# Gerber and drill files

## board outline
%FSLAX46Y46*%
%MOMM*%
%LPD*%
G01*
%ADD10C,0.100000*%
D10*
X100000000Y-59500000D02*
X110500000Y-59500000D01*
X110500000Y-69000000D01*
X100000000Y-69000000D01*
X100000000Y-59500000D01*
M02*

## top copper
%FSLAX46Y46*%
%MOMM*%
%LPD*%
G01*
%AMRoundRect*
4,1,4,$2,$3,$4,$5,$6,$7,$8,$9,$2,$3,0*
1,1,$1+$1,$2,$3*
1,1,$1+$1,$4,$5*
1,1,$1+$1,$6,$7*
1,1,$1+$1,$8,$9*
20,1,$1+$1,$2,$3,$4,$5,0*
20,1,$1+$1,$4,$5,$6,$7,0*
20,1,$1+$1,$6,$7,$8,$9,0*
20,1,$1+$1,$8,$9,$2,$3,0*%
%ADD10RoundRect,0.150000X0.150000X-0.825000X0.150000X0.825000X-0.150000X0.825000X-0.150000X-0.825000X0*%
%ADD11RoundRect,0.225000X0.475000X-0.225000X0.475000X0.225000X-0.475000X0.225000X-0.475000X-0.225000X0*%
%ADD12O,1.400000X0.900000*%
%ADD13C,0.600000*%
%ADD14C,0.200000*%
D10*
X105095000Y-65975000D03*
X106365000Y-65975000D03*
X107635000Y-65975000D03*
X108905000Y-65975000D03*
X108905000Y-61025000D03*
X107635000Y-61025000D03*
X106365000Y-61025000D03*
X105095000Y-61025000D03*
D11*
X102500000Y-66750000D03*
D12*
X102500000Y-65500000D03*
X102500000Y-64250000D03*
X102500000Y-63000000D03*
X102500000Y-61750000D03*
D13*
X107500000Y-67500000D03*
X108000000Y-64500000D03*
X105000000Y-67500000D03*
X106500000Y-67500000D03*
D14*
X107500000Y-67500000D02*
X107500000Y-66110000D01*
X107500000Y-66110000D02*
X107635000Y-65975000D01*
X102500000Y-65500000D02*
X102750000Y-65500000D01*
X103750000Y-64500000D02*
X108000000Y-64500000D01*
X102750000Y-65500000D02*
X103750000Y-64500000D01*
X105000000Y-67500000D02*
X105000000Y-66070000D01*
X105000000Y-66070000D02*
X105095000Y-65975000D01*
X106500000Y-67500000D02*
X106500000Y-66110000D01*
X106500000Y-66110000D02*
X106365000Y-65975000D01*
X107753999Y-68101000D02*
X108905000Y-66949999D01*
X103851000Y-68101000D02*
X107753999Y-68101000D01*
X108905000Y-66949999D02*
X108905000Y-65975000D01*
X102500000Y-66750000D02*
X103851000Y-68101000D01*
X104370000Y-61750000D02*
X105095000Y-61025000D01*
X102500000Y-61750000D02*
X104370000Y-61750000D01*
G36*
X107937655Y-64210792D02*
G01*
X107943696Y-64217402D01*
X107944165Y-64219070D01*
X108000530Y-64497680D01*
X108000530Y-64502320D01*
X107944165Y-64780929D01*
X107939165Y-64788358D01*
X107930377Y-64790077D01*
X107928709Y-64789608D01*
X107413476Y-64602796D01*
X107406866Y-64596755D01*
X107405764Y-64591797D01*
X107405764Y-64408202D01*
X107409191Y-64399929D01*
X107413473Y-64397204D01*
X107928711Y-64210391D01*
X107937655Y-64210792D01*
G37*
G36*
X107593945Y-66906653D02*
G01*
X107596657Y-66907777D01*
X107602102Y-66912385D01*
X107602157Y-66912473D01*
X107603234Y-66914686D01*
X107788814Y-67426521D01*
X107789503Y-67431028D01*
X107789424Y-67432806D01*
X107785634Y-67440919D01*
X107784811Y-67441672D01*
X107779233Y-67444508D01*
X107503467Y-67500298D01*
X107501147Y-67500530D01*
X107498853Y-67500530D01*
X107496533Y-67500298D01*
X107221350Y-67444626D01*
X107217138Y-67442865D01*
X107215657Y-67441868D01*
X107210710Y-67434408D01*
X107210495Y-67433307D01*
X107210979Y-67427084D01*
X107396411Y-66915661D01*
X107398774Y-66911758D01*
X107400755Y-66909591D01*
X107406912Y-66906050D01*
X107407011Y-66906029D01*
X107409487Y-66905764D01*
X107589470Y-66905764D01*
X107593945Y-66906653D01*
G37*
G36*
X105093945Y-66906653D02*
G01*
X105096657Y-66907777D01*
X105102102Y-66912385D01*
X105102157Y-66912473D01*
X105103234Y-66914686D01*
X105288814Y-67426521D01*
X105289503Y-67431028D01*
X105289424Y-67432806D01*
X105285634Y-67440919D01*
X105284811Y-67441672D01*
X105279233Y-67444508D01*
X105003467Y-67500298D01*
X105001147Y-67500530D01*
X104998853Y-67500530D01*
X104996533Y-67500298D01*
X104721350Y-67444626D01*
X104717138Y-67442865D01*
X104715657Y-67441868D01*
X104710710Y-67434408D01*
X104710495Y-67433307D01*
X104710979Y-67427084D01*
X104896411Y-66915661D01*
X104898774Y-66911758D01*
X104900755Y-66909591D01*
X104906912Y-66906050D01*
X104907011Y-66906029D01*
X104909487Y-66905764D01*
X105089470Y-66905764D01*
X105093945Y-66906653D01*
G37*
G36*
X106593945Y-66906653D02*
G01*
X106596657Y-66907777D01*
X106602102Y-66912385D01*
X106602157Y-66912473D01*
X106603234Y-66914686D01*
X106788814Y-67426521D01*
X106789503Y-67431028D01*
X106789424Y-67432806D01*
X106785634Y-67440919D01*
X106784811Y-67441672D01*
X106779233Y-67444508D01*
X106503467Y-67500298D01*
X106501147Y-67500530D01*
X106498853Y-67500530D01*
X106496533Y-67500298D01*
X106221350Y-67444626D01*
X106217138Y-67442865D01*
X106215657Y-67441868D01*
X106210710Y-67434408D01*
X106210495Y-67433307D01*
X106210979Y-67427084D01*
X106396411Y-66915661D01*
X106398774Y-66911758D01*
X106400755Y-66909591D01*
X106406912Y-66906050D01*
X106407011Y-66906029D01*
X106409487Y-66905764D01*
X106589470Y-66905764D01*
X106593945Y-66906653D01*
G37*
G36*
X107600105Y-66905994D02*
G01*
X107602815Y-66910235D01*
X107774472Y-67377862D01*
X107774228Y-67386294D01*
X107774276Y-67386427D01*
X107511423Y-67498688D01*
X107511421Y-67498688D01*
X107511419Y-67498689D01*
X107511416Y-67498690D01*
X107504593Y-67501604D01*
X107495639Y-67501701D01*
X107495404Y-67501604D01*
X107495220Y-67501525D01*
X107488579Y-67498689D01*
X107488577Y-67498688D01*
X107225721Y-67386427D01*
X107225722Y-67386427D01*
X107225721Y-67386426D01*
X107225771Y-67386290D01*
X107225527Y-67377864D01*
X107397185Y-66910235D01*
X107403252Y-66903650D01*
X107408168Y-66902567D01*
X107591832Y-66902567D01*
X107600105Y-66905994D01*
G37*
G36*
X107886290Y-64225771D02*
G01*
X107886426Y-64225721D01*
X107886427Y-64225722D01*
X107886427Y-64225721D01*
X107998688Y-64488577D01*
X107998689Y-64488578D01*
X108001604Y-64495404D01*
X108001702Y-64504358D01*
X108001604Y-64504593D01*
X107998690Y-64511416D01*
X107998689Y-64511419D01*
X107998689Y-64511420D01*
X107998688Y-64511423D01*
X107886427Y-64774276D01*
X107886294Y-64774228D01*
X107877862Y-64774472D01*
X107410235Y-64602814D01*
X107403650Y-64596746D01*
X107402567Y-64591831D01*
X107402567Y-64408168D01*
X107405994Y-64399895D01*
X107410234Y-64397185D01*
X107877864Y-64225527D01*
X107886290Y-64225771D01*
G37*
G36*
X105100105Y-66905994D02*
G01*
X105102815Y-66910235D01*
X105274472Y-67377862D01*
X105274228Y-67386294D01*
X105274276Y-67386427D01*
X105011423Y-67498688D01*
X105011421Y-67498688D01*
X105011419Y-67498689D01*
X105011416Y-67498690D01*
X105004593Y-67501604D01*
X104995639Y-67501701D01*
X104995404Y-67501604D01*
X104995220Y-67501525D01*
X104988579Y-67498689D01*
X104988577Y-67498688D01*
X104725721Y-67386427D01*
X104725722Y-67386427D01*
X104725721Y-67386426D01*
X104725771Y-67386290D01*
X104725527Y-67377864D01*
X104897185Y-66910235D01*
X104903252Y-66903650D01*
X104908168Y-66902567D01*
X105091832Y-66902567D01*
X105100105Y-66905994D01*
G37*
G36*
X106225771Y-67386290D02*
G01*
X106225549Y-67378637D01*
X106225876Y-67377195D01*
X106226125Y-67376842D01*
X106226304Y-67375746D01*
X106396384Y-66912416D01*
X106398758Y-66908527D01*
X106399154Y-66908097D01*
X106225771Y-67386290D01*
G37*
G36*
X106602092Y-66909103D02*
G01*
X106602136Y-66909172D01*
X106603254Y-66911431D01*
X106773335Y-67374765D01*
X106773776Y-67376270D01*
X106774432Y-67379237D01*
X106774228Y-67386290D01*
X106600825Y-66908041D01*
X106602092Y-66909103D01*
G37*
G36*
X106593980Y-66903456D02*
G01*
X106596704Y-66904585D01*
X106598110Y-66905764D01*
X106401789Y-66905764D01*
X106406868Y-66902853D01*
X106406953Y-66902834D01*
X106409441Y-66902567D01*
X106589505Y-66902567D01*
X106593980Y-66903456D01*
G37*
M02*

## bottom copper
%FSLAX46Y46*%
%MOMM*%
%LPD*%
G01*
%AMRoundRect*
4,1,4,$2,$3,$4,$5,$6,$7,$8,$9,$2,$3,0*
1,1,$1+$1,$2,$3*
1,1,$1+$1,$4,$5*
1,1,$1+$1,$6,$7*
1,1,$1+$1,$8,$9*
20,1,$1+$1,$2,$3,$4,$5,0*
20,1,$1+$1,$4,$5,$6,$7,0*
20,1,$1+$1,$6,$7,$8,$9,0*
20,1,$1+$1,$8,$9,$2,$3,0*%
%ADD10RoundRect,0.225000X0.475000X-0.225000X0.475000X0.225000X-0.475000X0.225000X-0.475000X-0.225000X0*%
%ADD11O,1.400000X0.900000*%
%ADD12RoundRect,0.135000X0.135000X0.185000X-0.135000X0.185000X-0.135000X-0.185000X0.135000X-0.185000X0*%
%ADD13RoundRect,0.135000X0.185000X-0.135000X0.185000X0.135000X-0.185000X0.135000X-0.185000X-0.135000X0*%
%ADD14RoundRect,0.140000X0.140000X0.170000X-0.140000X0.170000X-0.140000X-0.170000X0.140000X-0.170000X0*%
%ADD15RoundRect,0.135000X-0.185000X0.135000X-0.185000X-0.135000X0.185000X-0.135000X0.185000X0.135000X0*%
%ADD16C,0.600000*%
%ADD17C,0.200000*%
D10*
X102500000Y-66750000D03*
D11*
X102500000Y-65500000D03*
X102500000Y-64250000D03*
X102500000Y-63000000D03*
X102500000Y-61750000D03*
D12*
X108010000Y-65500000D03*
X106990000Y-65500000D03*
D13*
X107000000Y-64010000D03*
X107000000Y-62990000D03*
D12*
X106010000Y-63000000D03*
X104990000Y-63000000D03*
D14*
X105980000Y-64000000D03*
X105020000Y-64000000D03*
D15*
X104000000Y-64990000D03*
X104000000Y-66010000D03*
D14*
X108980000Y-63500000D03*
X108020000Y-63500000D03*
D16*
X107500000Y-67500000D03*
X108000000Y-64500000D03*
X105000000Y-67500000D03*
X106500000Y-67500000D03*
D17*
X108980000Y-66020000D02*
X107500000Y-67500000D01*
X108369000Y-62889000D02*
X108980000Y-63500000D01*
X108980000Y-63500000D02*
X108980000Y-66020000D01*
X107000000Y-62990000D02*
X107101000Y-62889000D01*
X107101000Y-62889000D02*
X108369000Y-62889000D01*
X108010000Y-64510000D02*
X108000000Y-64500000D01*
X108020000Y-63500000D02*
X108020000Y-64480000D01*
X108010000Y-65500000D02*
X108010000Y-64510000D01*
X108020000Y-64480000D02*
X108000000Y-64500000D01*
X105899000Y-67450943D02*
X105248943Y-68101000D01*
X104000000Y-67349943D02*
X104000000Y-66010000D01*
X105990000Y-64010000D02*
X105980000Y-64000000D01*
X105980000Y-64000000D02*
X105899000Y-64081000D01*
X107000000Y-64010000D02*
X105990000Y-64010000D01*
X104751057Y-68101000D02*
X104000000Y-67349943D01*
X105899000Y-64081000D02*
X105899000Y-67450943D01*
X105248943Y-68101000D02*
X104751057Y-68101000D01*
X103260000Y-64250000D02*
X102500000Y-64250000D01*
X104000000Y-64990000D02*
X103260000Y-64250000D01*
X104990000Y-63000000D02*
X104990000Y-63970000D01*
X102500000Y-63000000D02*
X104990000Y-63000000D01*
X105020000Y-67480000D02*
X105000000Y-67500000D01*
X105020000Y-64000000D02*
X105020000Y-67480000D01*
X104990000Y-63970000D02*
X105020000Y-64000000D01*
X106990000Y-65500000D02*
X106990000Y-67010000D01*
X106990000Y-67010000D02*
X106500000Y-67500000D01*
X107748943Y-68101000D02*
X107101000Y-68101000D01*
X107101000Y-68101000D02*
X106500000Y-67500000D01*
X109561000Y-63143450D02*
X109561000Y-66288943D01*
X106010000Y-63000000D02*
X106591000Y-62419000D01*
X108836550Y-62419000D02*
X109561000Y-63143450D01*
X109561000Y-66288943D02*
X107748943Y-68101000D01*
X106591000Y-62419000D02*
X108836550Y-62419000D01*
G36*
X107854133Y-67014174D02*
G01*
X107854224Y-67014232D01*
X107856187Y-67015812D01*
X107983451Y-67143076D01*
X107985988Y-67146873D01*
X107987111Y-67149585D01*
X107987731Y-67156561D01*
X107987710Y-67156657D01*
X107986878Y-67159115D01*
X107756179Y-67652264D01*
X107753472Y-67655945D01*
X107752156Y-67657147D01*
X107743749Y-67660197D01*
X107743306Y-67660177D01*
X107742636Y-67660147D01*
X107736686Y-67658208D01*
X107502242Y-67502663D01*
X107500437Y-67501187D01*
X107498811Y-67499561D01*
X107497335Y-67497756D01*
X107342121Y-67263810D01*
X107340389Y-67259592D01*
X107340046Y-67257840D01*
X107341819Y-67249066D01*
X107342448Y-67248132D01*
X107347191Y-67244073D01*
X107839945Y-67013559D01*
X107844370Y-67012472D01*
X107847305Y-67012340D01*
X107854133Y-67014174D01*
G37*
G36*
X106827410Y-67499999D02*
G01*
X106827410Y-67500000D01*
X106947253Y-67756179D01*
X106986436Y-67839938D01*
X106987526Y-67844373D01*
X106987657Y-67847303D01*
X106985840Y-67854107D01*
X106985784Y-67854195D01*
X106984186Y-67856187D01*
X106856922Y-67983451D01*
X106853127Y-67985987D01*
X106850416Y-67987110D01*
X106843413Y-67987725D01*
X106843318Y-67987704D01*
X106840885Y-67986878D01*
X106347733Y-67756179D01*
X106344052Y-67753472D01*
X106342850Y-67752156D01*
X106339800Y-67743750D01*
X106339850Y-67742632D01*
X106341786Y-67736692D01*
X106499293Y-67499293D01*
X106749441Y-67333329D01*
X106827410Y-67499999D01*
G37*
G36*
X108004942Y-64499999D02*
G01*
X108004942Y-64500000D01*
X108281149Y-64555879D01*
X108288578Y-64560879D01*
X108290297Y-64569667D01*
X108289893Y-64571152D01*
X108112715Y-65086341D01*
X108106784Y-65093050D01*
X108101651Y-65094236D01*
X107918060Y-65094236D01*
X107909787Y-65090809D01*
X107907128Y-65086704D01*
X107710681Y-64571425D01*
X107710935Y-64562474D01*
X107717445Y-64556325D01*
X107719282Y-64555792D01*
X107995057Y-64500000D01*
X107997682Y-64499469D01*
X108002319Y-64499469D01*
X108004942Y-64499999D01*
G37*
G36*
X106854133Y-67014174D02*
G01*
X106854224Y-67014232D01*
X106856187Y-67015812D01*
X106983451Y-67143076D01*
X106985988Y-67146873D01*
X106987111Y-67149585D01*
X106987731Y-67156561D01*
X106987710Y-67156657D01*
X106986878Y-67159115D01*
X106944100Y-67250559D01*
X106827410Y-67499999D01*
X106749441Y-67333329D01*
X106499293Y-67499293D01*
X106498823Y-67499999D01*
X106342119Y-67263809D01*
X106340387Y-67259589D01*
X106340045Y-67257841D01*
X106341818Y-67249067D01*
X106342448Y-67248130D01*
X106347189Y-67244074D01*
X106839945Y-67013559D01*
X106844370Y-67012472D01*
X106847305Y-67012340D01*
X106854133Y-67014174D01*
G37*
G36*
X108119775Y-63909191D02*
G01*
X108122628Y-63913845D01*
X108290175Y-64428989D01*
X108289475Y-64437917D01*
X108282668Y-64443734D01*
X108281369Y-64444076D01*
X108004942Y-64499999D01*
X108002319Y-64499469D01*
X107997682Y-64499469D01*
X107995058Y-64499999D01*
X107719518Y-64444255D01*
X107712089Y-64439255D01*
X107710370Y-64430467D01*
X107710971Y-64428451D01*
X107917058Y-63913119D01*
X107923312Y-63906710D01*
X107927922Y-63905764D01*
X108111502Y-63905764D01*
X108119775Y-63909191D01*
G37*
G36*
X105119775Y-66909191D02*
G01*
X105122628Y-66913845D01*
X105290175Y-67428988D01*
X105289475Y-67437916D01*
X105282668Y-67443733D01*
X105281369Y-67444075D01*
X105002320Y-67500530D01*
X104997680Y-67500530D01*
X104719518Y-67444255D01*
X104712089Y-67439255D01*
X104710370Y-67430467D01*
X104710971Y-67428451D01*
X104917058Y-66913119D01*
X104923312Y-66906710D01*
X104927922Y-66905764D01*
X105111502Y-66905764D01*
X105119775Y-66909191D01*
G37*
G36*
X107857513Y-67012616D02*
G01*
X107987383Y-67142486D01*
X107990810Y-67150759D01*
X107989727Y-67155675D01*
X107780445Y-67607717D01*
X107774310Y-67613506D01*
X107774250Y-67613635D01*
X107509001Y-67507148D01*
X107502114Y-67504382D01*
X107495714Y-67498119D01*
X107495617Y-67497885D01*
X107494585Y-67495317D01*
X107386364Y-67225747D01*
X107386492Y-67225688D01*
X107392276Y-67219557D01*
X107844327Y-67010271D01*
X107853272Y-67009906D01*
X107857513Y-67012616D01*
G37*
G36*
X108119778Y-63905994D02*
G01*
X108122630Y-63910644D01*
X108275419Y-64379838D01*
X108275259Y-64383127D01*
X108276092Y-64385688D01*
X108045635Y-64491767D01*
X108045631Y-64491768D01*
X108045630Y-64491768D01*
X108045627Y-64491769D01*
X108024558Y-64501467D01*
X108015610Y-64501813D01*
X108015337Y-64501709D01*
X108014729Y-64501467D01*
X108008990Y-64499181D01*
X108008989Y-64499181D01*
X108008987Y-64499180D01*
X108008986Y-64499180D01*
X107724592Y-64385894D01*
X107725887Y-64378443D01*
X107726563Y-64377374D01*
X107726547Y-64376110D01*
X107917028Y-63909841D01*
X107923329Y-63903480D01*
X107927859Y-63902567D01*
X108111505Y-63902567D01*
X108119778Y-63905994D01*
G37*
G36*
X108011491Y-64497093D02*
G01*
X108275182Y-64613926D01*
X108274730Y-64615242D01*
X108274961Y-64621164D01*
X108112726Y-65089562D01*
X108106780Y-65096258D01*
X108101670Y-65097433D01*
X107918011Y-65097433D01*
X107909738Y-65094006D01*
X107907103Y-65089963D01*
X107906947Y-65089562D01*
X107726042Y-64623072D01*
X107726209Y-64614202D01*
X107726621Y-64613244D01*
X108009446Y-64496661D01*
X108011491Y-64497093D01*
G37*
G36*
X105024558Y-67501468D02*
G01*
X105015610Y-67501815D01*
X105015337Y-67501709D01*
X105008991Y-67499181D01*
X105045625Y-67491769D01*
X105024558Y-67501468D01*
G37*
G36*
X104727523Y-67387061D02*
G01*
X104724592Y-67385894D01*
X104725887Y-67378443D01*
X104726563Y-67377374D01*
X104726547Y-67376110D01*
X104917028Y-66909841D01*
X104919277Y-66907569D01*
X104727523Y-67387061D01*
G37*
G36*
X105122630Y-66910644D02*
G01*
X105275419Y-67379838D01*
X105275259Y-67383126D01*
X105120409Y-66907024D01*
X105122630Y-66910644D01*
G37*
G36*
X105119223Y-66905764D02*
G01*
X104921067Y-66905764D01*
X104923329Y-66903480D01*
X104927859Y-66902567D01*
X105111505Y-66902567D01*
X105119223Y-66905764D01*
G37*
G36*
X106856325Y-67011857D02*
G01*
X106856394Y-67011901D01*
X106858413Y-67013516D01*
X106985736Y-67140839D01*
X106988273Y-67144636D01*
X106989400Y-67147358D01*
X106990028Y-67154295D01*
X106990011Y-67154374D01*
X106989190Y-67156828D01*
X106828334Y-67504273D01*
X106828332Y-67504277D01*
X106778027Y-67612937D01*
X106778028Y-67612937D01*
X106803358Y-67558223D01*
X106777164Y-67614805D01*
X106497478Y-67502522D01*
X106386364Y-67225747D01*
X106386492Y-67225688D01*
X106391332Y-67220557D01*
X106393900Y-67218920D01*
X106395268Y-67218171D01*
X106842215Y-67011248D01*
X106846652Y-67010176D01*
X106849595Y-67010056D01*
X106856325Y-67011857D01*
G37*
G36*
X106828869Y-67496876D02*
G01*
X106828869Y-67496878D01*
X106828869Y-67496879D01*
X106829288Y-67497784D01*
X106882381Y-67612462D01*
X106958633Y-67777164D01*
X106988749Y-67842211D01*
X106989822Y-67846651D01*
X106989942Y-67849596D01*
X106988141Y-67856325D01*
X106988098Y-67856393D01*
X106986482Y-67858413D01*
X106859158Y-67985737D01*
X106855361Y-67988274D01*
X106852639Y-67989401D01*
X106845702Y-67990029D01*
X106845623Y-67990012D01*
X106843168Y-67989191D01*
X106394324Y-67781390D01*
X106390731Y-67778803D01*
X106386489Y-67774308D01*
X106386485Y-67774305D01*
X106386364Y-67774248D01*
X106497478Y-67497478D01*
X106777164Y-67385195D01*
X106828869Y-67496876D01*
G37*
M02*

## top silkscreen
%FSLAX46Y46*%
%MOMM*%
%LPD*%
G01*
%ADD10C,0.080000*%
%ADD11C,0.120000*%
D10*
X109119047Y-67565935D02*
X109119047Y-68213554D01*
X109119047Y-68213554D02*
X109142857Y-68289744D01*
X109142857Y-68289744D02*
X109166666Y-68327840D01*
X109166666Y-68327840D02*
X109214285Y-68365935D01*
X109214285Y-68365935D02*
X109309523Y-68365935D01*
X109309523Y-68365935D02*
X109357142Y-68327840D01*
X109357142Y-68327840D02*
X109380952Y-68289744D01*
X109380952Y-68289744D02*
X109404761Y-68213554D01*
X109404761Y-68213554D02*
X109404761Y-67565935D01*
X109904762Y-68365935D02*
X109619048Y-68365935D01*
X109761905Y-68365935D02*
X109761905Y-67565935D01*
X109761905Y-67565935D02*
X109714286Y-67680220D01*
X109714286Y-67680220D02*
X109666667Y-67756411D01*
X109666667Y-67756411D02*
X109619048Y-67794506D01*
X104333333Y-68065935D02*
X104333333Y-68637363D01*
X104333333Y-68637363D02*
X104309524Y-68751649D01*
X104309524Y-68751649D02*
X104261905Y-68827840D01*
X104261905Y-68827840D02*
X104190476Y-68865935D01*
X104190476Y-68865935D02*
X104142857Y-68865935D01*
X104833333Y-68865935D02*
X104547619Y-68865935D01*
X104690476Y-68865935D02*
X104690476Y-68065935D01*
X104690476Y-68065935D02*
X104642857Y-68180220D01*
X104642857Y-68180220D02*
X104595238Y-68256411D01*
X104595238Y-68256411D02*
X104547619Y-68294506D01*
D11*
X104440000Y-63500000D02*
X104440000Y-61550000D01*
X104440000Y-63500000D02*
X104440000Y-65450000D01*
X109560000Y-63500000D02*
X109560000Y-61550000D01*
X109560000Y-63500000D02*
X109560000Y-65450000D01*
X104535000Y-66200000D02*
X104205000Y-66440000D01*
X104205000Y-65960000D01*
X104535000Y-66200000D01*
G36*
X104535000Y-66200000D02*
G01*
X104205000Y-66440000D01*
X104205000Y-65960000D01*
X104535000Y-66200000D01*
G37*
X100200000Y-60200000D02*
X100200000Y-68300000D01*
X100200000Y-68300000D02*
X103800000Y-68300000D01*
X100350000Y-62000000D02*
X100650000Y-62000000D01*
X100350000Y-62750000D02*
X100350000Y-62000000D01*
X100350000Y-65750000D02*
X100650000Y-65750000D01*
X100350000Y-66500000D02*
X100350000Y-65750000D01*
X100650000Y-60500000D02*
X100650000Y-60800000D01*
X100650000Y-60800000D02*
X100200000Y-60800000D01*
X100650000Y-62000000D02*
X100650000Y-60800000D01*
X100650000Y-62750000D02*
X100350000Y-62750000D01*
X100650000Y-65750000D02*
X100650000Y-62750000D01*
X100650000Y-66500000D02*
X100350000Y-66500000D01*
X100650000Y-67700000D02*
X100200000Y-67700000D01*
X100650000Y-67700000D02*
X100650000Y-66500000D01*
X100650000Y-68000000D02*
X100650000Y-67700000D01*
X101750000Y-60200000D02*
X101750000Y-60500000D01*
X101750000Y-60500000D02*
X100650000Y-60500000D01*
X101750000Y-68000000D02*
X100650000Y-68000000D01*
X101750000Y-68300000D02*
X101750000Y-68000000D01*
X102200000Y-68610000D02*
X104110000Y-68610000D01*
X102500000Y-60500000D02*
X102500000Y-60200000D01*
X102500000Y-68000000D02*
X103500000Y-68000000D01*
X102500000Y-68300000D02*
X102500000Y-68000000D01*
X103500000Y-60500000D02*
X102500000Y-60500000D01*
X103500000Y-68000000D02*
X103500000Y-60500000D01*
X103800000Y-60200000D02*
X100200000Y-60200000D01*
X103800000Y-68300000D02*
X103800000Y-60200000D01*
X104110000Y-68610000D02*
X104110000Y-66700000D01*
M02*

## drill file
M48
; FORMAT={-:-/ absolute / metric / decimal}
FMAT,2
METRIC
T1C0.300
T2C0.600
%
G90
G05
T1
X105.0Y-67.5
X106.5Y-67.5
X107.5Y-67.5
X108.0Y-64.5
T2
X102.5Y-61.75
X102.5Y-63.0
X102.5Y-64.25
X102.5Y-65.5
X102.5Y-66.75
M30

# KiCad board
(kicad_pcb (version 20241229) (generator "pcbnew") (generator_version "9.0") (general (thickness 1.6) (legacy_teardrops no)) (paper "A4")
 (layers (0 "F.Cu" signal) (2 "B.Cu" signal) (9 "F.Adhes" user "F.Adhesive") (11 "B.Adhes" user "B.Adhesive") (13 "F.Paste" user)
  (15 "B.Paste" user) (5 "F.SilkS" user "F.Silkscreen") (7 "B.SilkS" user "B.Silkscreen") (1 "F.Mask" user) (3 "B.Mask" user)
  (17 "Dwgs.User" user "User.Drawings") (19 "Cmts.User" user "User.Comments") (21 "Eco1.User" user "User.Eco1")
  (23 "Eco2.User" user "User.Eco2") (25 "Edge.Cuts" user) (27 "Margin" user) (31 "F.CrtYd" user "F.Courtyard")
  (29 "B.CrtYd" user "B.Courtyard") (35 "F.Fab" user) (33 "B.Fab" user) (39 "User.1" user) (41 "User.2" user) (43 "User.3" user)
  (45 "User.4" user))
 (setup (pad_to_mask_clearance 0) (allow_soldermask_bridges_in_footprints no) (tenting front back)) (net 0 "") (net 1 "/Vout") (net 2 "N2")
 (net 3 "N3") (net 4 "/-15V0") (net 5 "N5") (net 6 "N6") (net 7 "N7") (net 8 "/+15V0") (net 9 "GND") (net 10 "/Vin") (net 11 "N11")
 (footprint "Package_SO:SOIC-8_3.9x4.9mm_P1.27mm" (layer "F.Cu") (at 107 63.5 90)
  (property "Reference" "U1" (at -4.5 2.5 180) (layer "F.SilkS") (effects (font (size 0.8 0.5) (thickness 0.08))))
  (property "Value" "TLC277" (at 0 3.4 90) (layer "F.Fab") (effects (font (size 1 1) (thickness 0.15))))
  (fp_line (start 0 -2.56) (end 1.95 -2.56) (stroke (width 0.12) (type solid)) (layer "F.SilkS"))
  (fp_line (start 0 -2.56) (end -1.95 -2.56) (stroke (width 0.12) (type solid)) (layer "F.SilkS"))
  (fp_line (start 0 2.56) (end 1.95 2.56) (stroke (width 0.12) (type solid)) (layer "F.SilkS"))
  (fp_line (start 0 2.56) (end -1.95 2.56) (stroke (width 0.12) (type solid)) (layer "F.SilkS"))
  (fp_poly
   (pts (xy -2.7 -2.465) (xy -2.94 -2.795) (xy -2.46 -2.795) (xy -2.7 -2.465)) (stroke (width 0.12) (type solid)) (fill yes)
   (layer "F.SilkS"))
  (pad "1" smd roundrect (at -2.475 -1.905 90) (size 1.95 0.6) (layers "F.Cu" "F.Mask" "F.Paste") (roundrect_rratio 0.25) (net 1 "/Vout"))
  (pad "2" smd roundrect (at -2.475 -0.635 90) (size 1.95 0.6) (layers "F.Cu" "F.Mask" "F.Paste") (roundrect_rratio 0.25) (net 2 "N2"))
  (pad "3" smd roundrect (at -2.475 0.635 90) (size 1.95 0.6) (layers "F.Cu" "F.Mask" "F.Paste") (roundrect_rratio 0.25) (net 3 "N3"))
  (pad "4" smd roundrect (at -2.475 1.905 90) (size 1.95 0.6) (layers "F.Cu" "F.Mask" "F.Paste") (roundrect_rratio 0.25) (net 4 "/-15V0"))
  (pad "5" smd roundrect (at 2.475 1.905 90) (size 1.95 0.6) (layers "F.Cu" "F.Mask" "F.Paste") (roundrect_rratio 0.25) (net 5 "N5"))
  (pad "6" smd roundrect (at 2.475 0.635 90) (size 1.95 0.6) (layers "F.Cu" "F.Mask" "F.Paste") (roundrect_rratio 0.25) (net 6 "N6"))
  (pad "7" smd roundrect (at 2.475 -0.635 90) (size 1.95 0.6) (layers "F.Cu" "F.Mask" "F.Paste") (roundrect_rratio 0.25) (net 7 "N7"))
  (pad "8" smd roundrect (at 2.475 -1.905 90) (size 1.95 0.6) (layers "F.Cu" "F.Mask" "F.Paste") (roundrect_rratio 0.25) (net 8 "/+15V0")))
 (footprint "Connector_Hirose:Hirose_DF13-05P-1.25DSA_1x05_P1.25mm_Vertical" (layer "F.Cu") (at 102.5 66.75 90)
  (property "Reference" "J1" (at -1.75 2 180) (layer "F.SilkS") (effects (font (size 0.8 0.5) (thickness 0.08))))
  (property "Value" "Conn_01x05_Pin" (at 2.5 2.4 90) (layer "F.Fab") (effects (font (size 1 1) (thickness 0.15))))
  (fp_line (start 6.55 -2.3) (end -1.55 -2.3) (stroke (width 0.12) (type solid)) (layer "F.SilkS"))
  (fp_line (start -1.55 -2.3) (end -1.55 1.3) (stroke (width 0.12) (type solid)) (layer "F.SilkS"))
  (fp_line (start 4.75 -2.15) (end 4.75 -1.85) (stroke (width 0.12) (type solid)) (layer "F.SilkS"))
  (fp_line (start 4 -2.15) (end 4.75 -2.15) (stroke (width 0.12) (type solid)) (layer "F.SilkS"))
  (fp_line (start 1 -2.15) (end 1 -1.85) (stroke (width 0.12) (type solid)) (layer "F.SilkS"))
  (fp_line (start 0.25 -2.15) (end 1 -2.15) (stroke (width 0.12) (type solid)) (layer "F.SilkS"))
  (fp_line (start 6.25 -1.85) (end 5.95 -1.85) (stroke (width 0.12) (type solid)) (layer "F.SilkS"))
  (fp_line (start 5.95 -1.85) (end 5.95 -2.3) (stroke (width 0.12) (type solid)) (layer "F.SilkS"))
  (fp_line (start 4.75 -1.85) (end 5.95 -1.85) (stroke (width 0.12) (type solid)) (layer "F.SilkS"))
  (fp_line (start 4 -1.85) (end 4 -2.15) (stroke (width 0.12) (type solid)) (layer "F.SilkS"))
  (fp_line (start 1 -1.85) (end 4 -1.85) (stroke (width 0.12) (type solid)) (layer "F.SilkS"))
  (fp_line (start 0.25 -1.85) (end 0.25 -2.15) (stroke (width 0.12) (type solid)) (layer "F.SilkS"))
  (fp_line (start -0.95 -1.85) (end -0.95 -2.3) (stroke (width 0.12) (type solid)) (layer "F.SilkS"))
  (fp_line (start -0.95 -1.85) (end 0.25 -1.85) (stroke (width 0.12) (type solid)) (layer "F.SilkS"))
  (fp_line (start -1.25 -1.85) (end -0.95 -1.85) (stroke (width 0.12) (type solid)) (layer "F.SilkS"))
  (fp_line (start 6.55 -0.75) (end 6.25 -0.75) (stroke (width 0.12) (type solid)) (layer "F.SilkS"))
  (fp_line (start 6.25 -0.75) (end 6.25 -1.85) (stroke (width 0.12) (type solid)) (layer "F.SilkS"))
  (fp_line (start -1.25 -0.75) (end -1.25 -1.85) (stroke (width 0.12) (type solid)) (layer "F.SilkS"))
  (fp_line (start -1.55 -0.75) (end -1.25 -0.75) (stroke (width 0.12) (type solid)) (layer "F.SilkS"))
  (fp_line (start -1.86 -0.3) (end -1.86 1.61) (stroke (width 0.12) (type solid)) (layer "F.SilkS"))
  (fp_line (start 6.25 0) (end 6.55 0) (stroke (width 0.12) (type solid)) (layer "F.SilkS"))
  (fp_line (start -1.25 0) (end -1.25 1) (stroke (width 0.12) (type solid)) (layer "F.SilkS"))
  (fp_line (start -1.55 0) (end -1.25 0) (stroke (width 0.12) (type solid)) (layer "F.SilkS"))
  (fp_line (start 6.25 1) (end 6.25 0) (stroke (width 0.12) (type solid)) (layer "F.SilkS"))
  (fp_line (start -1.25 1) (end 6.25 1) (stroke (width 0.12) (type solid)) (layer "F.SilkS"))
  (fp_line (start 6.55 1.3) (end 6.55 -2.3) (stroke (width 0.12) (type solid)) (layer "F.SilkS"))
  (fp_line (start -1.55 1.3) (end 6.55 1.3) (stroke (width 0.12) (type solid)) (layer "F.SilkS"))
  (fp_line (start -1.86 1.61) (end 0.05 1.61) (stroke (width 0.12) (type solid)) (layer "F.SilkS"))
  (pad "1" thru_hole roundrect (at 0 0 90) (size 0.9 1.4) (drill 0.6) (layers "*.Cu" "*.Mask") (remove_unused_layers no)
   (roundrect_rratio 0.25) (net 4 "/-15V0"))
  (pad "2" thru_hole oval (at 1.25 0 90) (size 0.9 1.4) (drill 0.6) (layers "*.Cu" "*.Mask") (remove_unused_layers no) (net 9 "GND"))
  (pad "3" thru_hole oval (at 2.5 0 90) (size 0.9 1.4) (drill 0.6) (layers "*.Cu" "*.Mask") (remove_unused_layers no) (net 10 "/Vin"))
  (pad "4" thru_hole oval (at 3.75 0 90) (size 0.9 1.4) (drill 0.6) (layers "*.Cu" "*.Mask") (remove_unused_layers no) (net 1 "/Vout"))
  (pad "5" thru_hole oval (at 5 0 90) (size 0.9 1.4) (drill 0.6) (layers "*.Cu" "*.Mask") (remove_unused_layers no) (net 8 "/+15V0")))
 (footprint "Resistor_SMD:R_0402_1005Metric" (layer "B.Cu") (at 107.5 65.5 180)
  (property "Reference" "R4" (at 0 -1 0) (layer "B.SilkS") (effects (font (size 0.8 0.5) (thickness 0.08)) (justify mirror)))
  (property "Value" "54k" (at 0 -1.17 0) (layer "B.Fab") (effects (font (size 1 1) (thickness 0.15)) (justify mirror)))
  (pad "1" smd roundrect (at -0.51 0 180) (size 0.54 0.64) (layers "B.Cu" "B.Mask" "B.Paste") (roundrect_rratio 0.25) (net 9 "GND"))
  (pad "2" smd roundrect (at 0.51 0 180) (size 0.54 0.64) (layers "B.Cu" "B.Mask" "B.Paste") (roundrect_rratio 0.25) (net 2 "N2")))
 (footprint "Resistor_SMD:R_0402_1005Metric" (layer "B.Cu") (at 107 63.5 90)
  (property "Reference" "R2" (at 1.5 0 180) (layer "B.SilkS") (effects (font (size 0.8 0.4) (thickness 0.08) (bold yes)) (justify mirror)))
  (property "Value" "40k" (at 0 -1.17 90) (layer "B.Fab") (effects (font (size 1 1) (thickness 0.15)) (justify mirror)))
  (pad "1" smd roundrect (at -0.51 0 90) (size 0.54 0.64) (layers "B.Cu" "B.Mask" "B.Paste") (roundrect_rratio 0.25) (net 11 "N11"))
  (pad "2" smd roundrect (at 0.51 0 90) (size 0.54 0.64) (layers "B.Cu" "B.Mask" "B.Paste") (roundrect_rratio 0.25) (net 3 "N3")))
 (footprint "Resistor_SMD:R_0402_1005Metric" (layer "B.Cu") (at 105.5 63 180)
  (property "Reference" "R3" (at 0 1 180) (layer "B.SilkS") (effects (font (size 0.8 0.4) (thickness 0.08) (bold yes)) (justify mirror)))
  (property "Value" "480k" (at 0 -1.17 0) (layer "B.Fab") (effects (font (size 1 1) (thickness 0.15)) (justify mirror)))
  (pad "1" smd roundrect (at -0.51 0 180) (size 0.54 0.64) (layers "B.Cu" "B.Mask" "B.Paste") (roundrect_rratio 0.25) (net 2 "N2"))
  (pad "2" smd roundrect (at 0.51 0 180) (size 0.54 0.64) (layers "B.Cu" "B.Mask" "B.Paste") (roundrect_rratio 0.25) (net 1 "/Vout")))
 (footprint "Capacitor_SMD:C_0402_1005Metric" (layer "B.Cu") (at 105.5 64 180)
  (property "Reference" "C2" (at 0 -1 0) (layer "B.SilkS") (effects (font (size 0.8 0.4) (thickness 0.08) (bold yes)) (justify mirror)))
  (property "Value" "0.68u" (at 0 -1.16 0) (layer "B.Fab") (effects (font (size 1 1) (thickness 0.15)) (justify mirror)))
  (pad "1" smd roundrect (at -0.48 0 180) (size 0.56 0.62) (layers "B.Cu" "B.Mask" "B.Paste") (roundrect_rratio 0.25) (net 11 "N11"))
  (pad "2" smd roundrect (at 0.48 0 180) (size 0.56 0.62) (layers "B.Cu" "B.Mask" "B.Paste") (roundrect_rratio 0.25) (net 1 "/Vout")))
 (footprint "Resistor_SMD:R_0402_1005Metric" (layer "B.Cu") (at 104 65.5 -90)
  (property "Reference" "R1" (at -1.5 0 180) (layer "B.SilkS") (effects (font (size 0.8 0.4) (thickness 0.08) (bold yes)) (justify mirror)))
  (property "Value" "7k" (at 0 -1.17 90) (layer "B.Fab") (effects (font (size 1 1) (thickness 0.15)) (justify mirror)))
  (pad "1" smd roundrect (at -0.51 0 270) (size 0.54 0.64) (layers "B.Cu" "B.Mask" "B.Paste") (roundrect_rratio 0.25) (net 10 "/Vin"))
  (pad "2" smd roundrect (at 0.51 0 270) (size 0.54 0.64) (layers "B.Cu" "B.Mask" "B.Paste") (roundrect_rratio 0.25) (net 11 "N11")))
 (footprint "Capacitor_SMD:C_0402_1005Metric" (layer "B.Cu") (at 108.5 63.5 180)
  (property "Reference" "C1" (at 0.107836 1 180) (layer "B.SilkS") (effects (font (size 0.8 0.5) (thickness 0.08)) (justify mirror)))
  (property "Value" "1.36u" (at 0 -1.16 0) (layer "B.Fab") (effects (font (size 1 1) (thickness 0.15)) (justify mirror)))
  (pad "1" smd roundrect (at -0.48 0 180) (size 0.56 0.62) (layers "B.Cu" "B.Mask" "B.Paste") (roundrect_rratio 0.25) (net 3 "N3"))
  (pad "2" smd roundrect (at 0.48 0 180) (size 0.56 0.62) (layers "B.Cu" "B.Mask" "B.Paste") (roundrect_rratio 0.25) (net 9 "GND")))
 (gr_rect (start 100 59.5) (end 110.5 69) (stroke (width 0.1) (type solid)) (fill no) (layer "Edge.Cuts"))
 (segment (start 107.5 67.5) (end 107.5 66.11) (width 0.2) (layer "F.Cu") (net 3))
 (segment (start 107.5 66.11) (end 107.635 65.975) (width 0.2) (layer "F.Cu") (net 3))
 (via (at 107.5 67.5) (size 0.6) (drill 0.3) (layers "F.Cu" "B.Cu") (free yes)
  (teardrops (best_length_ratio 0.5) (max_length 1) (best_width_ratio 1) (max_width 2) (curved_edges no) (filter_ratio 0.9) (enabled yes)
   (allow_two_segments yes) (prefer_zone_connections yes))
  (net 3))
 (segment (start 108.98 66.02) (end 107.5 67.5) (width 0.2) (layer "B.Cu") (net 3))
 (segment (start 108.369 62.889) (end 108.98 63.5) (width 0.2) (layer "B.Cu") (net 3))
 (segment (start 108.98 63.5) (end 108.98 66.02) (width 0.2) (layer "B.Cu") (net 3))
 (segment (start 107 62.99) (end 107.101 62.889) (width 0.2) (layer "B.Cu") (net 3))
 (segment (start 107.101 62.889) (end 108.369 62.889) (width 0.2) (layer "B.Cu") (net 3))
 (segment (start 102.5 65.5) (end 102.75 65.5) (width 0.2) (layer "F.Cu") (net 9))
 (segment (start 103.75 64.5) (end 108 64.5) (width 0.2) (layer "F.Cu") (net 9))
 (segment (start 102.75 65.5) (end 103.75 64.5) (width 0.2) (layer "F.Cu") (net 9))
 (via (at 108 64.5) (size 0.6) (drill 0.3) (layers "F.Cu" "B.Cu") (free yes)
  (teardrops (best_length_ratio 0.5) (max_length 1) (best_width_ratio 1) (max_width 2) (curved_edges no) (filter_ratio 0.9) (enabled yes)
   (allow_two_segments yes) (prefer_zone_connections yes))
  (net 9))
 (segment (start 108.01 64.51) (end 108 64.5) (width 0.2) (layer "B.Cu") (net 9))
 (segment (start 108.02 63.5) (end 108.02 64.48) (width 0.2) (layer "B.Cu") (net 9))
 (segment (start 108.01 65.5) (end 108.01 64.51) (width 0.2) (layer "B.Cu") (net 9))
 (segment (start 108.02 64.48) (end 108 64.5) (width 0.2) (layer "B.Cu") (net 9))
 (segment (start 105.899 67.450943) (end 105.248943 68.101) (width 0.2) (layer "B.Cu") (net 11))
 (segment (start 104 67.349943) (end 104 66.01) (width 0.2) (layer "B.Cu") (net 11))
 (segment (start 105.99 64.01) (end 105.98 64) (width 0.2) (layer "B.Cu") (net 11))
 (segment (start 105.98 64) (end 105.899 64.081) (width 0.2) (layer "B.Cu") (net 11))
 (segment (start 107 64.01) (end 105.99 64.01) (width 0.2) (layer "B.Cu") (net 11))
 (segment (start 104.751057 68.101) (end 104 67.349943) (width 0.2) (layer "B.Cu") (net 11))
 (segment (start 105.899 64.081) (end 105.899 67.450943) (width 0.2) (layer "B.Cu") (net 11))
 (segment (start 105.248943 68.101) (end 104.751057 68.101) (width 0.2) (layer "B.Cu") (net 11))
 (segment (start 103.26 64.25) (end 102.5 64.25) (width 0.2) (layer "B.Cu") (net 10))
 (segment (start 104 64.99) (end 103.26 64.25) (width 0.2) (layer "B.Cu") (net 10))
 (segment (start 105 67.5) (end 105 66.07) (width 0.2) (layer "F.Cu") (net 1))
 (segment (start 105 66.07) (end 105.095 65.975) (width 0.2) (layer "F.Cu") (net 1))
 (via (at 105 67.5) (size 0.6) (drill 0.3) (layers "F.Cu" "B.Cu") (free yes)
  (teardrops (best_length_ratio 0.5) (max_length 1) (best_width_ratio 1) (max_width 2) (curved_edges no) (filter_ratio 0.9) (enabled yes)
   (allow_two_segments yes) (prefer_zone_connections yes))
  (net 1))
 (segment (start 104.99 63) (end 104.99 63.97) (width 0.2) (layer "B.Cu") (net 1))
 (segment (start 102.5 63) (end 104.99 63) (width 0.2) (layer "B.Cu") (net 1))
 (segment (start 105.02 67.48) (end 105 67.5) (width 0.2) (layer "B.Cu") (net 1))
 (segment (start 105.02 64) (end 105.02 67.48) (width 0.2) (layer "B.Cu") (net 1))
 (segment (start 104.99 63.97) (end 105.02 64) (width 0.2) (layer "B.Cu") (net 1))
 (segment (start 106.5 67.5) (end 106.5 66.11) (width 0.2) (layer "F.Cu") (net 2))
 (segment (start 106.5 66.11) (end 106.365 65.975) (width 0.2) (layer "F.Cu") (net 2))
 (via (at 106.5 67.5) (size 0.6) (drill 0.3) (layers "F.Cu" "B.Cu") (free yes)
  (teardrops (best_length_ratio 0.5) (max_length 1) (best_width_ratio 1) (max_width 2) (curved_edges no) (filter_ratio 0.9) (enabled yes)
   (allow_two_segments yes) (prefer_zone_connections yes))
  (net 2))
 (segment (start 106.99 65.5) (end 106.99 67.01) (width 0.2) (layer "B.Cu") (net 2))
 (segment (start 106.99 67.01) (end 106.5 67.5) (width 0.2) (layer "B.Cu") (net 2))
 (segment (start 107.748943 68.101) (end 107.101 68.101) (width 0.2) (layer "B.Cu") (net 2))
 (segment (start 107.101 68.101) (end 106.5 67.5) (width 0.2) (layer "B.Cu") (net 2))
 (segment (start 109.561 63.14345) (end 109.561 66.288943) (width 0.2) (layer "B.Cu") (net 2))
 (segment (start 106.01 63) (end 106.591 62.419) (width 0.2) (layer "B.Cu") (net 2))
 (segment (start 108.83655 62.419) (end 109.561 63.14345) (width 0.2) (layer "B.Cu") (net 2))
 (segment (start 109.561 66.288943) (end 107.748943 68.101) (width 0.2) (layer "B.Cu") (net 2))
 (segment (start 106.591 62.419) (end 108.83655 62.419) (width 0.2) (layer "B.Cu") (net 2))
 (segment (start 107.753999 68.101) (end 108.905 66.949999) (width 0.2) (layer "F.Cu") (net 4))
 (segment (start 103.851 68.101) (end 107.753999 68.101) (width 0.2) (layer "F.Cu") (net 4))
 (segment (start 108.905 66.949999) (end 108.905 65.975) (width 0.2) (layer "F.Cu") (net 4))
 (segment (start 102.5 66.75) (end 103.851 68.101) (width 0.2) (layer "F.Cu") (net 4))
 (segment (start 104.37 61.75) (end 105.095 61.025) (width 0.2) (layer "F.Cu") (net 8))
 (segment (start 102.5 61.75) (end 104.37 61.75) (width 0.2) (layer "F.Cu") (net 8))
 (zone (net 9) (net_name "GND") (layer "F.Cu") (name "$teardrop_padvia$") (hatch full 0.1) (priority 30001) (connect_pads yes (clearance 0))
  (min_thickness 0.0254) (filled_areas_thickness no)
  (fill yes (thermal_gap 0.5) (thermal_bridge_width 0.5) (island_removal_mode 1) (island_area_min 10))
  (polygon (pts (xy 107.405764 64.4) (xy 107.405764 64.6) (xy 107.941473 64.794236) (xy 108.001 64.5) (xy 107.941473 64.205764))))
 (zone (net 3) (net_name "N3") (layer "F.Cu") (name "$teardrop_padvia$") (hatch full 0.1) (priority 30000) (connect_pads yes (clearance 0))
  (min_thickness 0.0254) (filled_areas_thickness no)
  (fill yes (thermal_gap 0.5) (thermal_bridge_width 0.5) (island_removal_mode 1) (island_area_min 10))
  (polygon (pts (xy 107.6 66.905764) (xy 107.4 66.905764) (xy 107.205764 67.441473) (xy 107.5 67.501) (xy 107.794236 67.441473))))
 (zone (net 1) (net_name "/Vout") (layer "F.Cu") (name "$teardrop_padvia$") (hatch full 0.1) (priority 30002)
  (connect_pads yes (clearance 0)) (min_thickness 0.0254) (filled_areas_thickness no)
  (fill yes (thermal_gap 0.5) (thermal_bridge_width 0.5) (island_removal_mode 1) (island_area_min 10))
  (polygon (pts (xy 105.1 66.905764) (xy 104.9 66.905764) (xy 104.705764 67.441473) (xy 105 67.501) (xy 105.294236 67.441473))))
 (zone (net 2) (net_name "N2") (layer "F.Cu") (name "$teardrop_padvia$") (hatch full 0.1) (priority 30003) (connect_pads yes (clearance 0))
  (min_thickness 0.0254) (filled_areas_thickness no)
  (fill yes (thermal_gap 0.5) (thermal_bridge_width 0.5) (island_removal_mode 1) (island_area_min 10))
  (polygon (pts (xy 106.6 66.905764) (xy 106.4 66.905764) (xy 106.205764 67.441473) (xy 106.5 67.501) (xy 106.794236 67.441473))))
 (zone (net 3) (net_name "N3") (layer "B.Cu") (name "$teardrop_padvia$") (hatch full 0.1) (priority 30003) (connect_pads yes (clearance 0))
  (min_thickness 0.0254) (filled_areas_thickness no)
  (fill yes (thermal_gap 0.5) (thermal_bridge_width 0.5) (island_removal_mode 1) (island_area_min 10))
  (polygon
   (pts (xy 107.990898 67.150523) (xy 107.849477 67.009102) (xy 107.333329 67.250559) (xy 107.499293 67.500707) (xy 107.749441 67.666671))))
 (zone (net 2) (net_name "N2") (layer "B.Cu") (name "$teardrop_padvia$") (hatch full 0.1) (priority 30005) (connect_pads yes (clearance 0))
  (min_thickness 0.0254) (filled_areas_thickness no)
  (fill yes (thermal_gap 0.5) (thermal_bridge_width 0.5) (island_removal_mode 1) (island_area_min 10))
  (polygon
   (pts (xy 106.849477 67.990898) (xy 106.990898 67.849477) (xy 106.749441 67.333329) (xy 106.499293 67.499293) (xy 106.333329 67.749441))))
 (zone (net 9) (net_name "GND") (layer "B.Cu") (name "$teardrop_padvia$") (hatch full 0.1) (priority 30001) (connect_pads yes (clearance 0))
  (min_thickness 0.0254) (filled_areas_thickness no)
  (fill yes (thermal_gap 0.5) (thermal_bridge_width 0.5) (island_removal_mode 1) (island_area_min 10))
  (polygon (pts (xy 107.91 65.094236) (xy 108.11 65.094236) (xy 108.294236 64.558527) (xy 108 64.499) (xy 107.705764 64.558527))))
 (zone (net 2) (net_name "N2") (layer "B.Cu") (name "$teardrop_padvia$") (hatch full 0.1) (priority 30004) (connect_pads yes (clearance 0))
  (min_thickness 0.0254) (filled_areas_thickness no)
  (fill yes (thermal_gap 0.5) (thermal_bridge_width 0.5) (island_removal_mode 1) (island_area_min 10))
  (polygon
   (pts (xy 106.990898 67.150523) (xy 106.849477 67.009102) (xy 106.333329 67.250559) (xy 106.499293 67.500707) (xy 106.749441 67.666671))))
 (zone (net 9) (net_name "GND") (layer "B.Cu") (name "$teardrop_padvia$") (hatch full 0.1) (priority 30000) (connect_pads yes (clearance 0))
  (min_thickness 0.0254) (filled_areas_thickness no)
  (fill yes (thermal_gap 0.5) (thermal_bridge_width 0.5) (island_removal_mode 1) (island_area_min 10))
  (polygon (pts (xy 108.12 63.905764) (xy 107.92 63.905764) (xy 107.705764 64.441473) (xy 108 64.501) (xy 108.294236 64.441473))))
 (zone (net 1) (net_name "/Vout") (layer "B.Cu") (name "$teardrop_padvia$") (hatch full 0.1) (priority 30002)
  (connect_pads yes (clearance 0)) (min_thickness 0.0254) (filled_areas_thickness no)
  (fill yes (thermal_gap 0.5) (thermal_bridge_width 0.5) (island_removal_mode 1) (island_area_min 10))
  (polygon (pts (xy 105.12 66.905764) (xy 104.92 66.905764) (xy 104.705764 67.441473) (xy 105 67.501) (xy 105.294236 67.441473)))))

